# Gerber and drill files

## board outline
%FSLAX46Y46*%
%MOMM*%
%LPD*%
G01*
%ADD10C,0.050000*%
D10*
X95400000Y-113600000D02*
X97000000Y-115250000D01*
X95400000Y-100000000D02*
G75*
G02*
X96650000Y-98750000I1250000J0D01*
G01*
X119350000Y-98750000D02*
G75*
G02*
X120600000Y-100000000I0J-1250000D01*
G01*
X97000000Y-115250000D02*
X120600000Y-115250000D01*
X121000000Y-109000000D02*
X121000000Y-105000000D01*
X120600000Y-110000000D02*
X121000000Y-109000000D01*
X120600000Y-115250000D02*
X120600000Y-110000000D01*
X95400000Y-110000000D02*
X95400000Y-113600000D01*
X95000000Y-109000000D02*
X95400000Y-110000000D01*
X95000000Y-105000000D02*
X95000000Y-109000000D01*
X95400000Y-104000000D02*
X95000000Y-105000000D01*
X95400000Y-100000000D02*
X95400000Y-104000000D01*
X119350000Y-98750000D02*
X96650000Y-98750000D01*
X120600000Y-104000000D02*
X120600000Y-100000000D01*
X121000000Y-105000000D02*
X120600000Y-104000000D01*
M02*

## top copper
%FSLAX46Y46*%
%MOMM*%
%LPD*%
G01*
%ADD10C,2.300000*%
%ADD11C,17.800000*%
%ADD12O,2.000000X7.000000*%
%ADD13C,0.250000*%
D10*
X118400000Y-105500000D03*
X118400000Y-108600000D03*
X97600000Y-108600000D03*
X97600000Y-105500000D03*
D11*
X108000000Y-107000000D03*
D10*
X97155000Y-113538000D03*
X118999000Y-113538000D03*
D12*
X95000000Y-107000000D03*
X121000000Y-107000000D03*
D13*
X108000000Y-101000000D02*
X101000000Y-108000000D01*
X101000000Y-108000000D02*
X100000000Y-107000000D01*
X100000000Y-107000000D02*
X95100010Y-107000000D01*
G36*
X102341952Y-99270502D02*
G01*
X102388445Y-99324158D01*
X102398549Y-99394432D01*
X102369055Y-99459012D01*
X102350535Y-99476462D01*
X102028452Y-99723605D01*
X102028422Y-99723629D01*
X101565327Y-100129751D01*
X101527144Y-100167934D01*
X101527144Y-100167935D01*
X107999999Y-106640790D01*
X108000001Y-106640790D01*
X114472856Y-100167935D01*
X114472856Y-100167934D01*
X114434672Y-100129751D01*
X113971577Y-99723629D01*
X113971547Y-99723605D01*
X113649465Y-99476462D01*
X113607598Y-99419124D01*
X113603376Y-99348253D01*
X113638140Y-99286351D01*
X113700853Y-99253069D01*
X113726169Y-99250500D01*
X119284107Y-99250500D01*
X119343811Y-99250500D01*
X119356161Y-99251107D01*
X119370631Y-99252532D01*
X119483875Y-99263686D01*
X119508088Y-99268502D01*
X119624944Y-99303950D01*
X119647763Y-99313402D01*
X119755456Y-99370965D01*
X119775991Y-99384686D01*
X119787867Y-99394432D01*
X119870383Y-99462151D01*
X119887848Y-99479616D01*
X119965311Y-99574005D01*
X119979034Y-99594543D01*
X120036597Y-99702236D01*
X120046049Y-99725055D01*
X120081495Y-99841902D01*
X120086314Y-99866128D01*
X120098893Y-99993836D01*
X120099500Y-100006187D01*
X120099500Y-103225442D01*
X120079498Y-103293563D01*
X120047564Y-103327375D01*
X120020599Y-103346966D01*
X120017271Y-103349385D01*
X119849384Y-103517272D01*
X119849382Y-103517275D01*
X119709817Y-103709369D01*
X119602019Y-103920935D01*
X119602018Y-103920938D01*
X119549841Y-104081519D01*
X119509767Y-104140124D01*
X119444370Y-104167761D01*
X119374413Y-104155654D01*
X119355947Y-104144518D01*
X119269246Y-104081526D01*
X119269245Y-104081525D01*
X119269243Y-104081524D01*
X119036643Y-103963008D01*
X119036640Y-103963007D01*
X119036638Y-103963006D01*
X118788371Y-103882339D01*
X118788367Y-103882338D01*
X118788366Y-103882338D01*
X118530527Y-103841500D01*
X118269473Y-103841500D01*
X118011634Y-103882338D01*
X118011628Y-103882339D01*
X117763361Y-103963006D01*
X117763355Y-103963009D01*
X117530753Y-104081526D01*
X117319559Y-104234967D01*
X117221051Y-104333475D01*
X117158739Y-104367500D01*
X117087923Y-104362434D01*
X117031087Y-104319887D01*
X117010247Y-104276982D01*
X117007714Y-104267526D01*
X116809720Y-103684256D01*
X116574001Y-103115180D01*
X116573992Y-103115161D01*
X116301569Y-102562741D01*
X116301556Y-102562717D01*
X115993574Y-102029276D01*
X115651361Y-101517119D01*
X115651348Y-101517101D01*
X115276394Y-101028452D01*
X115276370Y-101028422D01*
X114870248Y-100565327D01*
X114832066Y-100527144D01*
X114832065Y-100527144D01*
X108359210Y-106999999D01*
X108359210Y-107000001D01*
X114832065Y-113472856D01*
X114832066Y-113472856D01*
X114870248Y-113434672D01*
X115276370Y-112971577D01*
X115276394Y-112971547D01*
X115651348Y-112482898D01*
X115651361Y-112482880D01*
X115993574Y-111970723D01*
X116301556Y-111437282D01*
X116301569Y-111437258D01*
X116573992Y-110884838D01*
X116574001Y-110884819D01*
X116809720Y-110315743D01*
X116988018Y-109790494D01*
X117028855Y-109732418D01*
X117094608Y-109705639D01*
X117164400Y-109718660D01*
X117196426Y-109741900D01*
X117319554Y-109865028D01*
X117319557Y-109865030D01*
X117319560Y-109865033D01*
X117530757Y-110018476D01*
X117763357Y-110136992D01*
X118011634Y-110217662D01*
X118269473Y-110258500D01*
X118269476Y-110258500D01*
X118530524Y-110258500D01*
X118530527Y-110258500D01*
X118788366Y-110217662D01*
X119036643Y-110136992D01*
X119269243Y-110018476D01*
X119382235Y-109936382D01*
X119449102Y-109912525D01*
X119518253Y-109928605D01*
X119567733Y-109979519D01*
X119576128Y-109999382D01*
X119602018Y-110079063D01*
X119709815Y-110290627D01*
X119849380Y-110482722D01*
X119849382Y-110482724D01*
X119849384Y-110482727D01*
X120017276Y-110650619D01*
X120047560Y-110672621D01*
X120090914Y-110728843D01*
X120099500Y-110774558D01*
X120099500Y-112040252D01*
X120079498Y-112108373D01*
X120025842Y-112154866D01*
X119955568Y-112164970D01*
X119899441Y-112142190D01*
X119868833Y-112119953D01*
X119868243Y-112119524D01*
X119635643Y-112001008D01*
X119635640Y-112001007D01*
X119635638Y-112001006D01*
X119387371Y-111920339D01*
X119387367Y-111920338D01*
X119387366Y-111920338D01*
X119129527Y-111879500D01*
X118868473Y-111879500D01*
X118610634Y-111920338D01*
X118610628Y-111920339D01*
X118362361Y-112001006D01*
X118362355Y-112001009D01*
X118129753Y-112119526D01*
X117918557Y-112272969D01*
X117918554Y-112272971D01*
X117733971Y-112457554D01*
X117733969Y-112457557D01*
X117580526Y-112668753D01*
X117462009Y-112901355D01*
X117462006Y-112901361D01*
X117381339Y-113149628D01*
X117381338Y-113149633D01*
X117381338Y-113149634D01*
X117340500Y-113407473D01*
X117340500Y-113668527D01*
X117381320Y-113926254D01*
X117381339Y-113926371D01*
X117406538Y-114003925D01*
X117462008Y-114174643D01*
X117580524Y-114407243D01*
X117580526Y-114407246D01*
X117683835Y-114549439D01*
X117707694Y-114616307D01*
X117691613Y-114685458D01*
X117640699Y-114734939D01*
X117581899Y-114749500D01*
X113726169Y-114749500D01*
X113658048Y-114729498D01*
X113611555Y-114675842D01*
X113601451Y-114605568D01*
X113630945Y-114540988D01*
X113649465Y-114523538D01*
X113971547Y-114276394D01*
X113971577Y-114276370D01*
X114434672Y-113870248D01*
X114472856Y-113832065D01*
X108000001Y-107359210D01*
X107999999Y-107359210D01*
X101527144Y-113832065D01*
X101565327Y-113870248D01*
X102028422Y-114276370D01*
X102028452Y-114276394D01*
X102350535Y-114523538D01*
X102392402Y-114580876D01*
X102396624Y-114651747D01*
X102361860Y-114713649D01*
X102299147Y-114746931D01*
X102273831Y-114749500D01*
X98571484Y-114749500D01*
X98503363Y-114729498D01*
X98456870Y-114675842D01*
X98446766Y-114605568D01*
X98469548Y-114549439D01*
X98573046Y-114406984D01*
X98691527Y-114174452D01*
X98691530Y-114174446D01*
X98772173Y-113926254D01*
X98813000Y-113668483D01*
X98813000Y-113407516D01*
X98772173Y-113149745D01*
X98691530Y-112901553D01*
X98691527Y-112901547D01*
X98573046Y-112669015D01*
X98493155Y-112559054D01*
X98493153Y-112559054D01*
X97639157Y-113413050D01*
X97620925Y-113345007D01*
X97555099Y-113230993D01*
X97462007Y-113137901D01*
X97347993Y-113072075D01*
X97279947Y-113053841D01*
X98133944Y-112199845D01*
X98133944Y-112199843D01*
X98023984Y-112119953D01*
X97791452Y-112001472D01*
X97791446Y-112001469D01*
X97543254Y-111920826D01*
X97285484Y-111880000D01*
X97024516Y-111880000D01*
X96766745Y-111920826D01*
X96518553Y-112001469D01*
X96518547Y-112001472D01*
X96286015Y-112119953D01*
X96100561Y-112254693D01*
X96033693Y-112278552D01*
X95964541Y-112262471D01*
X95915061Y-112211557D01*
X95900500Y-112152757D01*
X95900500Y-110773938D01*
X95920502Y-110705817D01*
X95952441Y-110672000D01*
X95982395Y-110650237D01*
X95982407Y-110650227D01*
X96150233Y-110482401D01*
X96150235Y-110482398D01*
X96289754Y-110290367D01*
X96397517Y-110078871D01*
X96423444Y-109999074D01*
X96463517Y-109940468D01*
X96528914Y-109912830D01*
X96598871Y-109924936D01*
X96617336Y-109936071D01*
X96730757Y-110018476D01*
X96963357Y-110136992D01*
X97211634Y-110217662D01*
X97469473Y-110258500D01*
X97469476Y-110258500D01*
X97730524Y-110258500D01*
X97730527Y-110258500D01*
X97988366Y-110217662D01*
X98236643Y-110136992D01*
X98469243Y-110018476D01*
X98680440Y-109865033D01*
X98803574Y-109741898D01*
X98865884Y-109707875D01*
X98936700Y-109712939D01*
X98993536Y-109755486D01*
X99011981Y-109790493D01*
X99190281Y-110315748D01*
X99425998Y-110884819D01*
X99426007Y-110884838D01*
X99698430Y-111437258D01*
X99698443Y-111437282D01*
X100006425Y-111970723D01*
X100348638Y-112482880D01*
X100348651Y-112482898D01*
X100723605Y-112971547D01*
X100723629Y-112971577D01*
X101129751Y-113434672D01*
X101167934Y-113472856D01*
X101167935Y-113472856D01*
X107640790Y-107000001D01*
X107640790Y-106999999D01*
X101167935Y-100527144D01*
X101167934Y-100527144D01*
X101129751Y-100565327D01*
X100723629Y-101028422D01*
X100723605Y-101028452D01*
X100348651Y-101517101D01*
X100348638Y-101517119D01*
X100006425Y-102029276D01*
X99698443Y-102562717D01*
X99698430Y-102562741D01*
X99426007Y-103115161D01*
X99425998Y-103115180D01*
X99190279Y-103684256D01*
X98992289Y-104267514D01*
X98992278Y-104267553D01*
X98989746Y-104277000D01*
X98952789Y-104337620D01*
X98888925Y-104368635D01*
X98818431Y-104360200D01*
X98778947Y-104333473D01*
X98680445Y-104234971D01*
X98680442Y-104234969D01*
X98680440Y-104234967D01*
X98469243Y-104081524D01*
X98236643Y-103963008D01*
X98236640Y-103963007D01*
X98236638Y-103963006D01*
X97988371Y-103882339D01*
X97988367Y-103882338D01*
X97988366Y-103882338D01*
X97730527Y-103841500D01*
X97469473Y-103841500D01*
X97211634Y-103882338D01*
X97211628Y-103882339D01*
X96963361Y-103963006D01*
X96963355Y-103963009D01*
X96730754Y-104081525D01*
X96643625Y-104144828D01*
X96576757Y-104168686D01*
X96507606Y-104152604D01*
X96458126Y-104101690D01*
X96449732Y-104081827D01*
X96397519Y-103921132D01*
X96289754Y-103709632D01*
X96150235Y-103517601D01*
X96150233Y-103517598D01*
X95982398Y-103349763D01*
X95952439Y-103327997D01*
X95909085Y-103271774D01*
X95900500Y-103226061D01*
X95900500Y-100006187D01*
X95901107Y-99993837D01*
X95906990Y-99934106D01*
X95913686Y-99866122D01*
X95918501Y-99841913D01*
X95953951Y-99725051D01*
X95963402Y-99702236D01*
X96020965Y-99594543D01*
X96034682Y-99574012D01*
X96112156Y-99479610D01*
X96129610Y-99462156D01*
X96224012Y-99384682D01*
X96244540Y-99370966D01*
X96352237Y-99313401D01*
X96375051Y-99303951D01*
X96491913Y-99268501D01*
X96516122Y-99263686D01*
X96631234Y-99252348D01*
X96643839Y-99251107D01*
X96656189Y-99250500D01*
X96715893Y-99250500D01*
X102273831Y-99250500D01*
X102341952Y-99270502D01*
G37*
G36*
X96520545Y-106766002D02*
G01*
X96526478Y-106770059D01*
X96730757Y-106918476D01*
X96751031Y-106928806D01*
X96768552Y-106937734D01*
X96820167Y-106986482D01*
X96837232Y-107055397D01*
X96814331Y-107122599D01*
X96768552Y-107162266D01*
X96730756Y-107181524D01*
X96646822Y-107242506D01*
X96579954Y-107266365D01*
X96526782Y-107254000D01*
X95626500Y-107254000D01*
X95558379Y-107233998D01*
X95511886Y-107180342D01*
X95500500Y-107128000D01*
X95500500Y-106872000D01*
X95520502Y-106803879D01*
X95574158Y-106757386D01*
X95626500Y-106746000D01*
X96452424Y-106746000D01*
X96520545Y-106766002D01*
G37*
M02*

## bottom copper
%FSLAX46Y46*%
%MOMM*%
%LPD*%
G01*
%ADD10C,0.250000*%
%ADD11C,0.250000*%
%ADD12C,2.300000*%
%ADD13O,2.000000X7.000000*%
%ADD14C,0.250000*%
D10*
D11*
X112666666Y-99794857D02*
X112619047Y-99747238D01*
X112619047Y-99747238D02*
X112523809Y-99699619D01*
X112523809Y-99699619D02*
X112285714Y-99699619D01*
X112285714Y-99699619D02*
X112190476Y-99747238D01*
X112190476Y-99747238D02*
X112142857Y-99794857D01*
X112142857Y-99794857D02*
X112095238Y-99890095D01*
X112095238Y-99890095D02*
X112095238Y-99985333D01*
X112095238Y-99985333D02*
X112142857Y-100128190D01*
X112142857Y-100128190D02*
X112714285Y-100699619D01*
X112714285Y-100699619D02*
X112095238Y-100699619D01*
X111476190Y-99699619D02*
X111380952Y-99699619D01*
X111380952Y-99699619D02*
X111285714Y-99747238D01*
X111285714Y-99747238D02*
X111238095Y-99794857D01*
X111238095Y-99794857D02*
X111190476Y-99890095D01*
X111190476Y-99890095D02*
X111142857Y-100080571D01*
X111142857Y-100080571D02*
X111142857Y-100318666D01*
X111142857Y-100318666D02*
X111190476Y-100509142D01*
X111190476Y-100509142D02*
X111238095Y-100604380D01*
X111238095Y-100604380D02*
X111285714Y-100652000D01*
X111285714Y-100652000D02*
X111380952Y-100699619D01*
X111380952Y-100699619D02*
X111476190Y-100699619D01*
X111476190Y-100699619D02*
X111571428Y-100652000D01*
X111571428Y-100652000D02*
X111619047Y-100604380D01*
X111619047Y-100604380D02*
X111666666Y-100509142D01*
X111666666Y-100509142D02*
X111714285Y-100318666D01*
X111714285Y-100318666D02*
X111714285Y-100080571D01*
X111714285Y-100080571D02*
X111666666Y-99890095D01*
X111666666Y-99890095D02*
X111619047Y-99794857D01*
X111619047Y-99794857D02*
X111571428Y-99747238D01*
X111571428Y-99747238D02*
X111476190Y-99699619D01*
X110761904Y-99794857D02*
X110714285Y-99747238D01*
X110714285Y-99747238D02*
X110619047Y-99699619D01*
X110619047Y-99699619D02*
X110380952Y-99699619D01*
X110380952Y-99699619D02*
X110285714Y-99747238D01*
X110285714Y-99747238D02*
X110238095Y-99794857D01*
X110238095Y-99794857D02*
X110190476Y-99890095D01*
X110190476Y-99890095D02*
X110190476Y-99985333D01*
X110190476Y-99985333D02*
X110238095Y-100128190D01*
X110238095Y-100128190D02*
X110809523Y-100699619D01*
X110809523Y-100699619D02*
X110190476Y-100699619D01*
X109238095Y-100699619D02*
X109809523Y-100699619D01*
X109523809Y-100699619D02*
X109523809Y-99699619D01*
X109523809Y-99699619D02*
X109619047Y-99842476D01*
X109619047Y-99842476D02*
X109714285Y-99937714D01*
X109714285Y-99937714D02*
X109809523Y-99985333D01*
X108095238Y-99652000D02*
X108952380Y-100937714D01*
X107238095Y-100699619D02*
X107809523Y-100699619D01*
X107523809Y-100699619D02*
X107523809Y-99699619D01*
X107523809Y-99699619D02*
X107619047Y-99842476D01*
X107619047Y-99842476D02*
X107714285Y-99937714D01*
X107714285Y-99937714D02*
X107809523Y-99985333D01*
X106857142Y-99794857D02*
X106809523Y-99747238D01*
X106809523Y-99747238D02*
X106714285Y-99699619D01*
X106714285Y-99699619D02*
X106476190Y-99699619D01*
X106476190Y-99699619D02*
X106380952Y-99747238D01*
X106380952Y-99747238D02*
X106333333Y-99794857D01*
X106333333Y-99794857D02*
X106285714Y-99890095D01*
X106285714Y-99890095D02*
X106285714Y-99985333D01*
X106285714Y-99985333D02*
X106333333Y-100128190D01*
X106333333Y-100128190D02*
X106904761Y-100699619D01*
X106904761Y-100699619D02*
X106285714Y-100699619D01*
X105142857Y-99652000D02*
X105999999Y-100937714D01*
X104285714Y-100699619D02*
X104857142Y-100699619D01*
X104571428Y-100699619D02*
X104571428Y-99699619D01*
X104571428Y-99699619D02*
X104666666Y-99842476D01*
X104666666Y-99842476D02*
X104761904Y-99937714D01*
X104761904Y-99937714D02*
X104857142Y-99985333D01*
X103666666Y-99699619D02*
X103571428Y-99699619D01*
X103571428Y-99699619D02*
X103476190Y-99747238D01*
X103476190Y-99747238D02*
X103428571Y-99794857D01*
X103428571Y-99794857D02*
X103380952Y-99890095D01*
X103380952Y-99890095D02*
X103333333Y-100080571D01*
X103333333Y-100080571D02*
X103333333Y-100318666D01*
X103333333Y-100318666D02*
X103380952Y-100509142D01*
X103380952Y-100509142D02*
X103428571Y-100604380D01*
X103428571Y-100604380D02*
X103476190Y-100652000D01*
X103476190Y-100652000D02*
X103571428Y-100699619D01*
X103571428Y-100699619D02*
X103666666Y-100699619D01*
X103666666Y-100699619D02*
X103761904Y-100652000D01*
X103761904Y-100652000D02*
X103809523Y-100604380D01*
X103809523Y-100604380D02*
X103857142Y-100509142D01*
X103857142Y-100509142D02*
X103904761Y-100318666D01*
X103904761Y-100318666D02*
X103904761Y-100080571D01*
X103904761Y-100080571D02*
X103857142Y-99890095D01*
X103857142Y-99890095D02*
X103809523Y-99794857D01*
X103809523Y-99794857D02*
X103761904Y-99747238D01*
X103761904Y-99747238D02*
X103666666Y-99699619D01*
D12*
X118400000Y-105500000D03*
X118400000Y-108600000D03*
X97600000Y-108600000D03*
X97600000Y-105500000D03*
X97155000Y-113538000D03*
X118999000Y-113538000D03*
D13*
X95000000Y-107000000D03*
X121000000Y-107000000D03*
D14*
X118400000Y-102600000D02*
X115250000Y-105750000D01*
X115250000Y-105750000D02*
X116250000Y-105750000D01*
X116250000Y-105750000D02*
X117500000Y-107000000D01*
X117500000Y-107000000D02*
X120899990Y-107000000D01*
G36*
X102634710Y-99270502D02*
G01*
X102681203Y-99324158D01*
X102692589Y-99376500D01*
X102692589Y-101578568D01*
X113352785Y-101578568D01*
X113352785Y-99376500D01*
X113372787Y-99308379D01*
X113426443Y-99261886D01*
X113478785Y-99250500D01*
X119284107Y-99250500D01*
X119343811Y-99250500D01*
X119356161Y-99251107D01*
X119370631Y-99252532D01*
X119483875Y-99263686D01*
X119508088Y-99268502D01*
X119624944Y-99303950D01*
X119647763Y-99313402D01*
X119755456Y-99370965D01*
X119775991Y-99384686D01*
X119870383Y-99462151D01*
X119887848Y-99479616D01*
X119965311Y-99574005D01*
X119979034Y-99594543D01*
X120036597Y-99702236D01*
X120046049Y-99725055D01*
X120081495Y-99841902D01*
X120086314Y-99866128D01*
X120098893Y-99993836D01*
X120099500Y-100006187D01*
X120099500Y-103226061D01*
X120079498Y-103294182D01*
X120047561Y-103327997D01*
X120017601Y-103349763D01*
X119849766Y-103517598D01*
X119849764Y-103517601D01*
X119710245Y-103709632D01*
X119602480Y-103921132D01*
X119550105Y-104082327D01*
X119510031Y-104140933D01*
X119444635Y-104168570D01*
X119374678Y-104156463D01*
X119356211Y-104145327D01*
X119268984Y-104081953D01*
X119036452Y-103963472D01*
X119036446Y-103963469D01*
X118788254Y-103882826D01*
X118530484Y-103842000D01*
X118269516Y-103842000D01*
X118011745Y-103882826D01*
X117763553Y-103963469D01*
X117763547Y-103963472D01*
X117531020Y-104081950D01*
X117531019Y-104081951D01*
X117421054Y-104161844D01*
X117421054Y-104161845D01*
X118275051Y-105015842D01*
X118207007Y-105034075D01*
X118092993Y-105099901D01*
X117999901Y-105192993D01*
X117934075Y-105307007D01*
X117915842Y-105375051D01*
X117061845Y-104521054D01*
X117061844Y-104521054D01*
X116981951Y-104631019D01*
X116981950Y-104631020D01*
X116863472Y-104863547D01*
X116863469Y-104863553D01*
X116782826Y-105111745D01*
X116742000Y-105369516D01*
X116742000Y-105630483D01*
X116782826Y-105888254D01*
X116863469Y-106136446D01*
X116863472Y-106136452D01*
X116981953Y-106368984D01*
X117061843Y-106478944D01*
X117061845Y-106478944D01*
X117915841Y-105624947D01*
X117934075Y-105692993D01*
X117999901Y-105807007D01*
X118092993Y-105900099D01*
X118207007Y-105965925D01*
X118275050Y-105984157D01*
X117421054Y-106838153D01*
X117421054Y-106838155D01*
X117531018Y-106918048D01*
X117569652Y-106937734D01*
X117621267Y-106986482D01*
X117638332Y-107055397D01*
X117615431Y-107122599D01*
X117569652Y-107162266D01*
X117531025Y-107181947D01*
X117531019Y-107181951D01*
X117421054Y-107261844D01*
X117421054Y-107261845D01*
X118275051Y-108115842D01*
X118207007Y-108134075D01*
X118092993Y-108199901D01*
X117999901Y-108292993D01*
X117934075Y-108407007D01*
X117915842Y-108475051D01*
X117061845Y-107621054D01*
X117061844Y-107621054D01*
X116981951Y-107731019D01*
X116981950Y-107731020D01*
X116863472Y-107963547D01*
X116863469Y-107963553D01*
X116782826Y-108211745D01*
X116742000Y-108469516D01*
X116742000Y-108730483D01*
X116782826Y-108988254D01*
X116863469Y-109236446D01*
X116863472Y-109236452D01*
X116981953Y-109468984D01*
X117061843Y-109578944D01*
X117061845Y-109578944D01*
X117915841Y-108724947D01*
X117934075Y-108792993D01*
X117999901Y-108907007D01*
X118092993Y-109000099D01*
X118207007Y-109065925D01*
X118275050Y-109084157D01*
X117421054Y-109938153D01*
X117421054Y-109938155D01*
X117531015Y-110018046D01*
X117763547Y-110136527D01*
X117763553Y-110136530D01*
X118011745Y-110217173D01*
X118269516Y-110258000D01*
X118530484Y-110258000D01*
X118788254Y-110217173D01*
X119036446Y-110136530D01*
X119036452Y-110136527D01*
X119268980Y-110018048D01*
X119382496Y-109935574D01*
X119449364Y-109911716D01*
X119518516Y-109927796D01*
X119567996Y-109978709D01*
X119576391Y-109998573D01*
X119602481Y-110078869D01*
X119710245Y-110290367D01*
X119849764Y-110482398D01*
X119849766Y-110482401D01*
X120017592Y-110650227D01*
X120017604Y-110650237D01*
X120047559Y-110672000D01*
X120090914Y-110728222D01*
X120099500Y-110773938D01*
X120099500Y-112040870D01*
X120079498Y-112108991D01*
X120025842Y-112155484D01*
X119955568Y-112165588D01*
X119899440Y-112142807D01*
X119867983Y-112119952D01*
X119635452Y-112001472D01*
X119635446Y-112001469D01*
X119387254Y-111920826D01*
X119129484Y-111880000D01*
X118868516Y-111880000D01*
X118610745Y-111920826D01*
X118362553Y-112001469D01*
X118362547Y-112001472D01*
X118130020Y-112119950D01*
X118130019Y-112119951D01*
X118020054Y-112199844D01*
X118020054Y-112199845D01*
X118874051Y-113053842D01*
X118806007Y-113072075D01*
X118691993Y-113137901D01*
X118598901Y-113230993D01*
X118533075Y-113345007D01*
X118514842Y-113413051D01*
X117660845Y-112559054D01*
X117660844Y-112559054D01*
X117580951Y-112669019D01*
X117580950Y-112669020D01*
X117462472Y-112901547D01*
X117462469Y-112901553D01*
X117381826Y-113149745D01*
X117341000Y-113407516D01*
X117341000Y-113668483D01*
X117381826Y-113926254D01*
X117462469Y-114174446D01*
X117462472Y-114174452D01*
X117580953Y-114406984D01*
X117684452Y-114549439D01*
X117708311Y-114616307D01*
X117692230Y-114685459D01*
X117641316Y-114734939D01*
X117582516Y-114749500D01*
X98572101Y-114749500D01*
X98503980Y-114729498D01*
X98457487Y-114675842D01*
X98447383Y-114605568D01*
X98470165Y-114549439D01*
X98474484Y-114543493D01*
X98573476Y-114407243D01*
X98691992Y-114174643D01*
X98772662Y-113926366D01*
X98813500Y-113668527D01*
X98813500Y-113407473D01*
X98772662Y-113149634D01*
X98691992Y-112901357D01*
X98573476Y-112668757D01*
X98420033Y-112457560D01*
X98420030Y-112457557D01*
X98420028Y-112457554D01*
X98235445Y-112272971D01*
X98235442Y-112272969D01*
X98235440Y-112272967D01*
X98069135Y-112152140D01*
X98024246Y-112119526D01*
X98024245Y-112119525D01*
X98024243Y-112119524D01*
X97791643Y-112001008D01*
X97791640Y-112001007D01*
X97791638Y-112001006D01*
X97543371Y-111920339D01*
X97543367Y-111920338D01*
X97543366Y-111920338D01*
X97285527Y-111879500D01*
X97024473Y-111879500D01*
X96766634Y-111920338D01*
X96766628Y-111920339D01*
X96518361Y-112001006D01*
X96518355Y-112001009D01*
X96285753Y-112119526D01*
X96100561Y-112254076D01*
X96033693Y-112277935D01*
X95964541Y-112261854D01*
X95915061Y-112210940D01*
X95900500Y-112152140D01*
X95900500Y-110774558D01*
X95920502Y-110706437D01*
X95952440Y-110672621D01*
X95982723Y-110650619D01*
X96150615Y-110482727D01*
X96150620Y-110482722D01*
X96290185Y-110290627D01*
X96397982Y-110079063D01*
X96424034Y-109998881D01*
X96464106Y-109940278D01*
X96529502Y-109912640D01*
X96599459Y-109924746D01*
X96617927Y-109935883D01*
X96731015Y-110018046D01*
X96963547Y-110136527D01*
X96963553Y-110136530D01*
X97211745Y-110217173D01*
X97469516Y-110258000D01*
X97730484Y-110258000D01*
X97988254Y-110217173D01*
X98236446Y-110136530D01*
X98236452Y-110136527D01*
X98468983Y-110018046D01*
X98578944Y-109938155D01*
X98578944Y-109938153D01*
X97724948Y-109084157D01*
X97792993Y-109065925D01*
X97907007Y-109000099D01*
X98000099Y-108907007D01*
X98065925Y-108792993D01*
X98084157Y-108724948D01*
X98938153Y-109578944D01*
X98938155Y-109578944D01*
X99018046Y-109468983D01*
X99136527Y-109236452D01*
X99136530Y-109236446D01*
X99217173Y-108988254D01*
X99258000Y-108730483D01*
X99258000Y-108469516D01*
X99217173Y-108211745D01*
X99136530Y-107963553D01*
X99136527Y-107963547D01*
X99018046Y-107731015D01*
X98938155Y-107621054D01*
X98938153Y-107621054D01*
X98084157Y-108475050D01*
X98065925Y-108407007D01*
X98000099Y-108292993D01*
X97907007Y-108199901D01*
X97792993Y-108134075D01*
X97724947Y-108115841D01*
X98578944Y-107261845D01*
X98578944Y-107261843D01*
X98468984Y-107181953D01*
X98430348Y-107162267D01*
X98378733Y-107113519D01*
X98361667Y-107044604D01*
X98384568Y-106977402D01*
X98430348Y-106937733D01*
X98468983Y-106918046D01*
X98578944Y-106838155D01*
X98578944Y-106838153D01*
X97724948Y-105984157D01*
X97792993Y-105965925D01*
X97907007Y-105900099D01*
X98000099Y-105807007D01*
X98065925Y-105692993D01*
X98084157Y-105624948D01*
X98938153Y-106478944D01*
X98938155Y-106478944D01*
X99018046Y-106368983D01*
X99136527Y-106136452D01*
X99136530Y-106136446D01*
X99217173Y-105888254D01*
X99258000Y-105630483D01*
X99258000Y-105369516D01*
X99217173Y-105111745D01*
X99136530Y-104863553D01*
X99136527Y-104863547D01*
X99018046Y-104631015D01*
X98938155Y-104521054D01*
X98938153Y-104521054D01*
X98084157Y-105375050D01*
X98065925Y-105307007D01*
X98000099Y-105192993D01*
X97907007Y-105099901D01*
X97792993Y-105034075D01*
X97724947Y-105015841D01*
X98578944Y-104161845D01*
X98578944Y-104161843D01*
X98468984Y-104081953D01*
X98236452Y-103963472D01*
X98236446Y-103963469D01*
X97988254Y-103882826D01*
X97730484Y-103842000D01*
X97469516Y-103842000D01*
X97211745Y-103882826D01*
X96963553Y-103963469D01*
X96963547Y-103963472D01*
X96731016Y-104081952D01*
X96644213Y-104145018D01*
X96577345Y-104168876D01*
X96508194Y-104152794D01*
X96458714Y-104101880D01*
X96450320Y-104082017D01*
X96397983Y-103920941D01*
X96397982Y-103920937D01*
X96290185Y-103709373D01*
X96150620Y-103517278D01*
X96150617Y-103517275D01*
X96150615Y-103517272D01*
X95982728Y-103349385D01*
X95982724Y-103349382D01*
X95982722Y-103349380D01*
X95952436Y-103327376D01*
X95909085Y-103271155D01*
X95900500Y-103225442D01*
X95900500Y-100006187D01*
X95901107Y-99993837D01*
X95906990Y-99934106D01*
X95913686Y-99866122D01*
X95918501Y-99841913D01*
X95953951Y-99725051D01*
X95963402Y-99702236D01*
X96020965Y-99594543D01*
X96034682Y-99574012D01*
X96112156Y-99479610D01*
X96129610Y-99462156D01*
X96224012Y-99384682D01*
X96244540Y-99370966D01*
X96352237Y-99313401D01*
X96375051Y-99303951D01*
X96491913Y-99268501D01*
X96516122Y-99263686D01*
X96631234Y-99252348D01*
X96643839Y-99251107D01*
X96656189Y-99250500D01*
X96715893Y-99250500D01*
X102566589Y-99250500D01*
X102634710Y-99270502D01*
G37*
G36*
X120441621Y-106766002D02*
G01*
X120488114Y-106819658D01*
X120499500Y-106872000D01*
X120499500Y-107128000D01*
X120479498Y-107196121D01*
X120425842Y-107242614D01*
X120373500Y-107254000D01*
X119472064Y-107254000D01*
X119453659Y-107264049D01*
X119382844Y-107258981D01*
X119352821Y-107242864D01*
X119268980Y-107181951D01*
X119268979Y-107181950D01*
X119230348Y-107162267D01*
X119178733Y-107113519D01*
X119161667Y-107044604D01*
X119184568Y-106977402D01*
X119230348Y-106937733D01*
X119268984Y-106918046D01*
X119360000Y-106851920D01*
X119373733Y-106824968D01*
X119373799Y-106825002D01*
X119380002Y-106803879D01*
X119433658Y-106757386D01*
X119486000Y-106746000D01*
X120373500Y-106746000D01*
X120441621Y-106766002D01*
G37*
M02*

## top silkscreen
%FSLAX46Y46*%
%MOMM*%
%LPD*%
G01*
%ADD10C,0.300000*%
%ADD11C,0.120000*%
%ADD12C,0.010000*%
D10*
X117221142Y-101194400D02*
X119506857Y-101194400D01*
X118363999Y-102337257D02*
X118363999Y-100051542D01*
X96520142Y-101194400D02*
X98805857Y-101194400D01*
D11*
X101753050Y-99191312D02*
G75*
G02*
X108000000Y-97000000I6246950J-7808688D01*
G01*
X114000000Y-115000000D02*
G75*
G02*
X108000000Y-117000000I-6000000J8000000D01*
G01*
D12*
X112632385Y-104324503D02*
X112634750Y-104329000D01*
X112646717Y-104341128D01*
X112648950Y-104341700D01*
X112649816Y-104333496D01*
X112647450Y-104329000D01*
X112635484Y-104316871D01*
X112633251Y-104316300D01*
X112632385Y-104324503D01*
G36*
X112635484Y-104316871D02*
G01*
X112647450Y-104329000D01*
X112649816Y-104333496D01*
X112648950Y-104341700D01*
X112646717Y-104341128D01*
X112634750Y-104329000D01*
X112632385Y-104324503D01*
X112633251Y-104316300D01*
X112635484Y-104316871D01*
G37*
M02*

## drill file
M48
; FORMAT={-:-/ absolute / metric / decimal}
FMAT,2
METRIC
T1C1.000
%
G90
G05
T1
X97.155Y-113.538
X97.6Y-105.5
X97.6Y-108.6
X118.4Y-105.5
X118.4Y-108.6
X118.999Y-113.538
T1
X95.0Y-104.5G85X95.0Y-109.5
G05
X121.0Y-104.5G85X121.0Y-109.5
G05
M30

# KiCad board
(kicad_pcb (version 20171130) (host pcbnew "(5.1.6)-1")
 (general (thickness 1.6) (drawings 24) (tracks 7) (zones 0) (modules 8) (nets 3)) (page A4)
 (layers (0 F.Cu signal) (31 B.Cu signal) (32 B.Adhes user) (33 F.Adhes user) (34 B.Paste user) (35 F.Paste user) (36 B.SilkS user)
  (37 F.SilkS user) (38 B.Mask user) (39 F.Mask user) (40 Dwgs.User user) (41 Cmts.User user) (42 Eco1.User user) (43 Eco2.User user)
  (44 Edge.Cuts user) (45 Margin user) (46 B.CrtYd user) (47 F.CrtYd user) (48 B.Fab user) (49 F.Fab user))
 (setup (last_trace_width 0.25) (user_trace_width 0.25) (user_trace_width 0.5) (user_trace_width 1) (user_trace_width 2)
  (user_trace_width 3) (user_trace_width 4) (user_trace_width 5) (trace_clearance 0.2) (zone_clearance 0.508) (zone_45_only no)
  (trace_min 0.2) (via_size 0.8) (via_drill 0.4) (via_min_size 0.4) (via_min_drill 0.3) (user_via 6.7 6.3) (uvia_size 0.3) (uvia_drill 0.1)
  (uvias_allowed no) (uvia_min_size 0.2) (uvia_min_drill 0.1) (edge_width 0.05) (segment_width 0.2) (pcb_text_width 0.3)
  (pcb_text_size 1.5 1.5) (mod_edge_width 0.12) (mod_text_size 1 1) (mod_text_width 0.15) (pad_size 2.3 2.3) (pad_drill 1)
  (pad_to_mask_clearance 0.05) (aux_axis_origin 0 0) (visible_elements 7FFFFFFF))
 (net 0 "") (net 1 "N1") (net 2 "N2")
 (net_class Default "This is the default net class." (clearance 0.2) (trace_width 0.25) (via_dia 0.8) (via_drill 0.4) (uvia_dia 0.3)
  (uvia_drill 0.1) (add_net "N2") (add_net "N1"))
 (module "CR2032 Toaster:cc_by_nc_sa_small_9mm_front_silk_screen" (layer B.Cu) (at 107.95 113.5 180)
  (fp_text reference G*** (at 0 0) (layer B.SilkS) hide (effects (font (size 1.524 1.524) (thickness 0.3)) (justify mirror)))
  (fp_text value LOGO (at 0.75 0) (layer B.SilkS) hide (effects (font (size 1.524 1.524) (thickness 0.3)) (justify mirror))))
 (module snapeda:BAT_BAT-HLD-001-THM (layer F.Cu) (at 108 107)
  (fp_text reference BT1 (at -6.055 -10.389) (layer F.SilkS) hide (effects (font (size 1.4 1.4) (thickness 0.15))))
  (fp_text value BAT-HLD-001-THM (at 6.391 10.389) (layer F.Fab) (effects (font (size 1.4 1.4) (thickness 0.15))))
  (pad P4 thru_hole circle (at 10.4 -1.5) (size 2.3 2.3) (drill 1) (layers *.Cu *.Mask) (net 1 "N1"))
  (pad P3 thru_hole circle (at 10.4 1.6) (size 2.3 2.3) (drill 1) (layers *.Cu *.Mask) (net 1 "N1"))
  (pad P2 thru_hole circle (at -10.4 1.6) (size 2.3 2.3) (drill 1) (layers *.Cu *.Mask) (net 1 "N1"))
  (pad P1 thru_hole circle (at -10.4 -1.5) (size 2.3 2.3) (drill 1) (layers *.Cu *.Mask) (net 1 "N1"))
  (pad N smd circle (at 0 0) (size 17.8 17.8) (layers F.Cu F.Mask) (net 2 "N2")))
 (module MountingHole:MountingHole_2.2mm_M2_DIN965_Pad (layer F.Cu) (at 97.155 113.538)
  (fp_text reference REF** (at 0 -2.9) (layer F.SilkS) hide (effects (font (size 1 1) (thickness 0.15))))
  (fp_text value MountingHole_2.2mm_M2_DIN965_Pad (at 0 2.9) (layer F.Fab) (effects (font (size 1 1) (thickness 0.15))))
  (pad 1 thru_hole circle (at 0 0) (size 2.3 2.3) (drill 1) (layers *.Cu *.Mask) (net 2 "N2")))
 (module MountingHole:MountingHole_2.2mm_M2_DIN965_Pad (layer F.Cu) (at 118.999 113.538)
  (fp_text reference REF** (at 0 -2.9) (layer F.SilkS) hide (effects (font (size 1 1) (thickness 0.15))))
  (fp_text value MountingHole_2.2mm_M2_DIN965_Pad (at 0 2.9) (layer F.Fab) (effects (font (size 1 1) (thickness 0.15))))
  (pad 1 thru_hole circle (at 0 0) (size 2.3 2.3) (drill 1) (layers *.Cu *.Mask) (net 1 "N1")))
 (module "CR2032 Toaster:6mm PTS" (layer F.Cu) (at 95 107)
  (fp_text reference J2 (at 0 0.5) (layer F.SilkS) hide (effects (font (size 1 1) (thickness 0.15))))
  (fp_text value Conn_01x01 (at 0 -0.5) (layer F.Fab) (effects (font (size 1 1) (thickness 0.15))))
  (pad 1 thru_hole oval (at 0 0) (size 2 7) (drill oval 1 6) (layers *.Cu *.Mask) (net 2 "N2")))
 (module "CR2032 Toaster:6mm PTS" (layer F.Cu) (at 121 107)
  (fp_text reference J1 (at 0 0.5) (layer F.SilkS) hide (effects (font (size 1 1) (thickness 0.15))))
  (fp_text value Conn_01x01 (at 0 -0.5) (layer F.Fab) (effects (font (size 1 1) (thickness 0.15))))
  (pad 1 thru_hole oval (at 0 0) (size 2 7) (drill oval 1 6) (layers *.Cu *.Mask) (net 1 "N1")))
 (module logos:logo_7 (layer F.Cu) (at 114 106.25)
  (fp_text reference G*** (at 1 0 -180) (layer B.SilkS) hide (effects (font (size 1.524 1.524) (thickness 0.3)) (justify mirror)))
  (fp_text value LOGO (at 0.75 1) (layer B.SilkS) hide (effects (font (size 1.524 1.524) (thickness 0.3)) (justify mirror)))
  (fp_poly
   (pts (xy -1.367615 -1.925497) (xy -1.36525 -1.921) (xy -1.353283 -1.908872) (xy -1.35105 -1.9083) (xy -1.350184 -1.916504)
    (xy -1.35255 -1.921) (xy -1.364516 -1.933129) (xy -1.366749 -1.9337) (xy -1.367615 -1.925497))
   (layer F.SilkS) (width 0.01)))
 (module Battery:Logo (layer F.Cu) (at 0 0)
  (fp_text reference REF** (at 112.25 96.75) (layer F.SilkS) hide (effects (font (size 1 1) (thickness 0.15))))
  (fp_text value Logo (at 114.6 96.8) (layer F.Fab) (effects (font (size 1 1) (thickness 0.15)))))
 (gr_line (start 95.4 113.6) (end 97 115.25) (layer Edge.Cuts) (width 0.05))
 (gr_arc (start 96.65 100) (end 96.65 98.75) (angle -90) (layer Edge.Cuts) (width 0.05))
 (gr_arc (start 119.35 100) (end 120.6 100) (angle -90) (layer Edge.Cuts) (width 0.05))
 (gr_line (start 97 115.25) (end 120.6 115.25) (layer Edge.Cuts) (width 0.05))
 (gr_line (start 121 109) (end 121 105) (layer Edge.Cuts) (width 0.05))
 (gr_line (start 120.6 110) (end 121 109) (layer Edge.Cuts) (width 0.05))
 (gr_line (start 120.6 115.25) (end 120.6 110) (layer Edge.Cuts) (width 0.05))
 (gr_line (start 95.4 110) (end 95.4 113.6) (layer Edge.Cuts) (width 0.05))
 (gr_line (start 95 109) (end 95.4 110) (layer Edge.Cuts) (width 0.05))
 (gr_line (start 95 105) (end 95 109) (layer Edge.Cuts) (width 0.05))
 (gr_line (start 95.4 104) (end 95 105) (layer Edge.Cuts) (width 0.05))
 (gr_line (start 95.4 100) (end 95.4 104) (layer Edge.Cuts) (width 0.05))
 (gr_line (start 119.35 98.75) (end 96.65 98.75) (layer Edge.Cuts) (width 0.05))
 (gr_line (start 120.6 104) (end 120.6 100) (layer Edge.Cuts) (width 0.05))
 (gr_line (start 121 105) (end 120.6 104) (layer Edge.Cuts) (width 0.05))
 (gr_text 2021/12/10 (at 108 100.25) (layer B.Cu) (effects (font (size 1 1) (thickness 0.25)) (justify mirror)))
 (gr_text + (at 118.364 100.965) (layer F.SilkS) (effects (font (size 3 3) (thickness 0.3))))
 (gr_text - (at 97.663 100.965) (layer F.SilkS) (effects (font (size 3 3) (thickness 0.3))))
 (gr_arc (start 108 107) (end 108 97) (angle -38.65980825) (layer F.SilkS) (width 0.12))
 (gr_arc (start 108 107) (end 108 117) (angle -36.86989765) (layer F.SilkS) (width 0.12))
 (segment (start 118.4 102.6) (end 115.25 105.75) (width 0.25) (layer B.Cu) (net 1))
 (segment (start 115.25 105.75) (end 116.25 105.75) (width 0.25) (layer B.Cu) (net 1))
 (segment (start 116.25 105.75) (end 117.5 107) (width 0.25) (layer B.Cu) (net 1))
 (segment (start 117.5 107) (end 120.89999 107) (width 0.25) (layer B.Cu) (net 1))
 (segment (start 108 101) (end 101 108) (width 0.25) (layer F.Cu) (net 2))
 (segment (start 101 108) (end 100 107) (width 0.25) (layer F.Cu) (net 2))
 (segment (start 100 107) (end 95.10001 107) (width 0.25) (layer F.Cu) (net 2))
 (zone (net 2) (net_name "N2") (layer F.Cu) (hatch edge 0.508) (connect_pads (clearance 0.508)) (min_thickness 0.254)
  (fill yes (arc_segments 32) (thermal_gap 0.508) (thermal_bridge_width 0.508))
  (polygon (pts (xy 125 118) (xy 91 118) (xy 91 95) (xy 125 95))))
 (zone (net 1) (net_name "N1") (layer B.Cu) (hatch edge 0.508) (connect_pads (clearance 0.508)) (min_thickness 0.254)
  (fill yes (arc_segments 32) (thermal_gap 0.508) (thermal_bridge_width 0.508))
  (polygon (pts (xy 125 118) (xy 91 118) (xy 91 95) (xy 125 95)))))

